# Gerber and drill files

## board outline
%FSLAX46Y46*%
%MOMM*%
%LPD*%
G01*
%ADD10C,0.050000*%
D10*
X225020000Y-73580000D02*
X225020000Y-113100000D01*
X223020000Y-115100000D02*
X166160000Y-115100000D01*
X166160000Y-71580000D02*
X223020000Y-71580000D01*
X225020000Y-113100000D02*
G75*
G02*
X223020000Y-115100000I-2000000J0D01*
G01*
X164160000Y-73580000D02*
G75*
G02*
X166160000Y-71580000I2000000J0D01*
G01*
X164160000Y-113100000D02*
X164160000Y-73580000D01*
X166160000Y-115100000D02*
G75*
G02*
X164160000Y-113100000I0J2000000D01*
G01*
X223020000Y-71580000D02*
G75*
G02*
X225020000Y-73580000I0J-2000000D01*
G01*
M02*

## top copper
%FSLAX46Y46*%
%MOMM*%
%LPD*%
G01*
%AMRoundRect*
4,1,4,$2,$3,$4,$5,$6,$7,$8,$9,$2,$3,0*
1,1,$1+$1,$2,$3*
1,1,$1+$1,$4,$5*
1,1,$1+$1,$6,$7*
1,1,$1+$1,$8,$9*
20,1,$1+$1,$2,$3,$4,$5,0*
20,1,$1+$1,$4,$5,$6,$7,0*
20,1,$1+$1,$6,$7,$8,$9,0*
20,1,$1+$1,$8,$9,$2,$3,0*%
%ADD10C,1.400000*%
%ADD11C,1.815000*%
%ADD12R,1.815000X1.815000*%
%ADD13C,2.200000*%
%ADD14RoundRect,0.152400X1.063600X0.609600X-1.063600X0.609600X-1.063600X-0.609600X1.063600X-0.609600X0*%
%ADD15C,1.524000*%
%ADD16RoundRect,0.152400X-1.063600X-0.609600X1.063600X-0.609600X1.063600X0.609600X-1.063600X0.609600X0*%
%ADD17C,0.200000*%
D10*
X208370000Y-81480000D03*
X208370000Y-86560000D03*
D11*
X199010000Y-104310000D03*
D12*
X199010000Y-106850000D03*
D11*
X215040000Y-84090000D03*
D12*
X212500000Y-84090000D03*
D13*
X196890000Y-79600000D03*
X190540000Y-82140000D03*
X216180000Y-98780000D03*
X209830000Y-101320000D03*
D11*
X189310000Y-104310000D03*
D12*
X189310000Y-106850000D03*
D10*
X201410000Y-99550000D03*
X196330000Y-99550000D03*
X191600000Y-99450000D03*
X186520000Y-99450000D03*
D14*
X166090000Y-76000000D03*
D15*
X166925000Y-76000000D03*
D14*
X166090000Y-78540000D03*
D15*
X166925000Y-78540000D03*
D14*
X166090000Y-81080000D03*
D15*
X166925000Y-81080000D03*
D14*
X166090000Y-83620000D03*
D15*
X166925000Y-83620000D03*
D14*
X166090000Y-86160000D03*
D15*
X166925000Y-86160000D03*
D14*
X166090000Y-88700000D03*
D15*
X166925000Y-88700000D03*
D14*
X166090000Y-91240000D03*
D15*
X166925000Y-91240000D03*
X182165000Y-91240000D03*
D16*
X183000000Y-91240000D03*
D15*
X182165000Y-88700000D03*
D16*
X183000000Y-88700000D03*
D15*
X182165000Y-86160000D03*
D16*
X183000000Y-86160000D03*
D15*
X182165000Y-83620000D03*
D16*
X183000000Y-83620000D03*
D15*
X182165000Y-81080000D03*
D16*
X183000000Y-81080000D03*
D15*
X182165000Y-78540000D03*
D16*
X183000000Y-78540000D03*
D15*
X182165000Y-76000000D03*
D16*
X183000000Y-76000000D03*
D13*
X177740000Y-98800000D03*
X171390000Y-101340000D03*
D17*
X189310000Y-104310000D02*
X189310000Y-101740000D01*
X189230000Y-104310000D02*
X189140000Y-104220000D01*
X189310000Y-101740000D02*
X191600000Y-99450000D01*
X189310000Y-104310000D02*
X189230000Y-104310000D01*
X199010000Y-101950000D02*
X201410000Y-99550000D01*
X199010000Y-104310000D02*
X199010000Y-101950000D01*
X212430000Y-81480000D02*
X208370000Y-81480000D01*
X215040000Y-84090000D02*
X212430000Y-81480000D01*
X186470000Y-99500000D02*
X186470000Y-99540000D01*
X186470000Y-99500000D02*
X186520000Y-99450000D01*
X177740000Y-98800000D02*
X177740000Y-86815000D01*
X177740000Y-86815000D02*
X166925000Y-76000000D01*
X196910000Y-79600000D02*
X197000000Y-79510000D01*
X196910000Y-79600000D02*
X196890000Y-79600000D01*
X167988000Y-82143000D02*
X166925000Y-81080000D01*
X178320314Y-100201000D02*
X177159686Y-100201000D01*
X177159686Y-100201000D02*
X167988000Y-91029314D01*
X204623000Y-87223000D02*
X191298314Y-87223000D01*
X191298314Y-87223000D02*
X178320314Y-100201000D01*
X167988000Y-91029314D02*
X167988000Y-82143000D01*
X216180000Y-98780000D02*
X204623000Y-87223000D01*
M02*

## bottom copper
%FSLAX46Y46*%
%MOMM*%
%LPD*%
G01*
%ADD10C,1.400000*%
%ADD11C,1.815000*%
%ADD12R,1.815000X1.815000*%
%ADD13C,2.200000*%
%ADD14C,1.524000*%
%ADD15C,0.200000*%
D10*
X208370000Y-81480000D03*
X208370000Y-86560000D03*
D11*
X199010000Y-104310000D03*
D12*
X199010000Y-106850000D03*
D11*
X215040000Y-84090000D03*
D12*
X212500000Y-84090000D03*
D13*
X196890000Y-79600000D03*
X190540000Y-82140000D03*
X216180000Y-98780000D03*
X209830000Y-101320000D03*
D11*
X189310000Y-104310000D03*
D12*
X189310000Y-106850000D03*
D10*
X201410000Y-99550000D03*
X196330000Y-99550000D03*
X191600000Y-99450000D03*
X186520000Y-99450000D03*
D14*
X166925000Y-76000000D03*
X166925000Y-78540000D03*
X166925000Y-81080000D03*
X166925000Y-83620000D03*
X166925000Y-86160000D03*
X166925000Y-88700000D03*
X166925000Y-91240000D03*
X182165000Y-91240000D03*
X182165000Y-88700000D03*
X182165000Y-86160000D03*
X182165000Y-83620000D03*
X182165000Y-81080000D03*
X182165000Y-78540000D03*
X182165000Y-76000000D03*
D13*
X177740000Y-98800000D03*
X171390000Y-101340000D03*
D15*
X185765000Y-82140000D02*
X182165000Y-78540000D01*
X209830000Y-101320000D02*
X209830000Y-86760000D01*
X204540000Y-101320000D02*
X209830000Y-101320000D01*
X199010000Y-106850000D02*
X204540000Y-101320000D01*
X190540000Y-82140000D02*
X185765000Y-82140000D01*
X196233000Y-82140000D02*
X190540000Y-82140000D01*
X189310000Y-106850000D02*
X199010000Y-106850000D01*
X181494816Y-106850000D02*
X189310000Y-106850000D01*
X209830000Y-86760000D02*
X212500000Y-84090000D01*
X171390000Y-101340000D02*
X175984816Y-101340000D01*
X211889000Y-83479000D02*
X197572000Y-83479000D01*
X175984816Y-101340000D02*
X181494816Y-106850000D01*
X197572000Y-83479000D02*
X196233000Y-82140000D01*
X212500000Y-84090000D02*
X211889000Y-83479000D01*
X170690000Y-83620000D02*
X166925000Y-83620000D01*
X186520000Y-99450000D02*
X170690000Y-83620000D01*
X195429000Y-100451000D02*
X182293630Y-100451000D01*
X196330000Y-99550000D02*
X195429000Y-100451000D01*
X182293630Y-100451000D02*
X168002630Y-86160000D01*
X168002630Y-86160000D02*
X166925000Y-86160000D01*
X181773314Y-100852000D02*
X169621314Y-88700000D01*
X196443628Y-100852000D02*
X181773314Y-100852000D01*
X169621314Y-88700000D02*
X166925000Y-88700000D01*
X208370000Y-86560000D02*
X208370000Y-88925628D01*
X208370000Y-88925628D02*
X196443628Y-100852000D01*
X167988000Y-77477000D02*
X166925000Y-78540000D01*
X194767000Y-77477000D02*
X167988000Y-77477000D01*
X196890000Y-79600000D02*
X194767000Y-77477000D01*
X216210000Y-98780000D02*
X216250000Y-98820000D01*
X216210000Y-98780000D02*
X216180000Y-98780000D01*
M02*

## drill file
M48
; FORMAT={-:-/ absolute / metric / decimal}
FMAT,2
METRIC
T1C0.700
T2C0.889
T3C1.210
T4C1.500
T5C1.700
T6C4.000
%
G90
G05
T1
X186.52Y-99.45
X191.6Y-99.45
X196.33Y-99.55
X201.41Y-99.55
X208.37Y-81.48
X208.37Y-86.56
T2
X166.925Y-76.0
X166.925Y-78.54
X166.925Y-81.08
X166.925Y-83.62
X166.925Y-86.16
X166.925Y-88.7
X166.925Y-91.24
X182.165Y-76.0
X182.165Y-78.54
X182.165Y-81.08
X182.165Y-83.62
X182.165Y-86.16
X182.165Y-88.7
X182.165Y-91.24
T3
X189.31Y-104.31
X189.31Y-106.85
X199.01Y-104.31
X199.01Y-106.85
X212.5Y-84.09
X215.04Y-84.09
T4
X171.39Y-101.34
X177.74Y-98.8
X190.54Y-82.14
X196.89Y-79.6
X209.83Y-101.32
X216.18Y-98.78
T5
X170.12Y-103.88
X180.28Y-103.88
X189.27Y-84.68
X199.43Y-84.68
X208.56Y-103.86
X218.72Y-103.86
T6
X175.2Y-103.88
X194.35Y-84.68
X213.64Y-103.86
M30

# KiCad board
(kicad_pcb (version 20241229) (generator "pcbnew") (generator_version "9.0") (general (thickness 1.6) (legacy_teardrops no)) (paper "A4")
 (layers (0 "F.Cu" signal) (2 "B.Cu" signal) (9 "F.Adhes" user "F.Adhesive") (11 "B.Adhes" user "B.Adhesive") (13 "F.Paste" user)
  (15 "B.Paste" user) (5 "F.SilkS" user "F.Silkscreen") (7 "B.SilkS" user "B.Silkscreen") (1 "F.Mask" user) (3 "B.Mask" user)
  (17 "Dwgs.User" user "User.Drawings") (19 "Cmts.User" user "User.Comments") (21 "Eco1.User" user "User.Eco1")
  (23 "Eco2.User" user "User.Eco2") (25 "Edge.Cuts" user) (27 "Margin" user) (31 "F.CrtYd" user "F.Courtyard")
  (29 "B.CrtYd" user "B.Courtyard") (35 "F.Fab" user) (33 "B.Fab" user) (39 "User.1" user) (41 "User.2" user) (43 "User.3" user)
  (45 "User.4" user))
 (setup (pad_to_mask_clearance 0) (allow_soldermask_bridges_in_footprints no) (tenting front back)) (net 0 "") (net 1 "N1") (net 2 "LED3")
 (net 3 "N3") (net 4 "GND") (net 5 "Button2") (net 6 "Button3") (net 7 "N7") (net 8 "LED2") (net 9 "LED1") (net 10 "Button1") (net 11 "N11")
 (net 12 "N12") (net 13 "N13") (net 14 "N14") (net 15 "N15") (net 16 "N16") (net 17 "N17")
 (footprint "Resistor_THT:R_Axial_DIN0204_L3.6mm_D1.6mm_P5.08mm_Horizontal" (layer "F.Cu") (at 208.37 81.48 -90)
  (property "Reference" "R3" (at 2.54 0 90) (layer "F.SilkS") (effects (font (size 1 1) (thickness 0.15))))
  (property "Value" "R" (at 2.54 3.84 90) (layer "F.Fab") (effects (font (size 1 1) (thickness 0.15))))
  (pad "1" thru_hole circle (at 0 0 270) (size 1.4 1.4) (drill 0.7) (layers "*.Cu" "*.Mask") (remove_unused_layers no) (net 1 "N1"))
  (pad "2" thru_hole circle (at 5.08 0 270) (size 1.4 1.4) (drill 0.7) (layers "*.Cu" "*.Mask") (remove_unused_layers no) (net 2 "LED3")))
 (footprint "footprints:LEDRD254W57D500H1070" (layer "F.Cu") (at 199.01 105.58 90)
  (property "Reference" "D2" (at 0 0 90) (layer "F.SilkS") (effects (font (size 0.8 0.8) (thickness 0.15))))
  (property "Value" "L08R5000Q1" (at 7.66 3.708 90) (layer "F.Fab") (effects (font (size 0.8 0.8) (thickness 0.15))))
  (pad "A" thru_hole circle (at 1.27 0 90) (size 1.815 1.815) (drill 1.21) (layers "*.Cu" "*.Mask") (remove_unused_layers no) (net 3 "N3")
   (solder_mask_margin 0.102))
  (pad "C" thru_hole rect (at -1.27 0 90) (size 1.815 1.815) (drill 1.21) (layers "*.Cu" "*.Mask") (remove_unused_layers no) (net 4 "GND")
   (solder_mask_margin 0.102)))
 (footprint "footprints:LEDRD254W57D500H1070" (layer "F.Cu") (at 213.77 84.09)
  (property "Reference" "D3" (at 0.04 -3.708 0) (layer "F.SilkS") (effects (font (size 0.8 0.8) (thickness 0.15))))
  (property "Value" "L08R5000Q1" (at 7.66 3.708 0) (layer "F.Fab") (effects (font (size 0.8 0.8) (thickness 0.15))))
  (pad "A" thru_hole circle (at 1.27 0) (size 1.815 1.815) (drill 1.21) (layers "*.Cu" "*.Mask") (remove_unused_layers no) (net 1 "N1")
   (solder_mask_margin 0.102))
  (pad "C" thru_hole rect (at -1.27 0) (size 1.815 1.815) (drill 1.21) (layers "*.Cu" "*.Mask") (remove_unused_layers no) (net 4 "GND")
   (solder_mask_margin 0.102)))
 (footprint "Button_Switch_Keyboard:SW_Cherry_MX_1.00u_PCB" (layer "F.Cu") (at 196.89 79.6)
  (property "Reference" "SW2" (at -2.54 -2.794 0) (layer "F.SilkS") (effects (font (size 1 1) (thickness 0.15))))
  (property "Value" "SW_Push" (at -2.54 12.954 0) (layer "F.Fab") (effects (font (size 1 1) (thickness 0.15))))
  (pad "" np_thru_hole circle (at -7.62 5.08) (size 1.7 1.7) (drill 1.7) (layers "*.Cu" "*.Mask"))
  (pad "" np_thru_hole circle (at -2.54 5.08) (size 4 4) (drill 4) (layers "*.Cu" "*.Mask"))
  (pad "" np_thru_hole circle (at 2.54 5.08) (size 1.7 1.7) (drill 1.7) (layers "*.Cu" "*.Mask"))
  (pad "1" thru_hole circle (at 0 0) (size 2.2 2.2) (drill 1.5) (layers "*.Cu" "*.Mask") (remove_unused_layers no) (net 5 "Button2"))
  (pad "2" thru_hole circle (at -6.35 2.54) (size 2.2 2.2) (drill 1.5) (layers "*.Cu" "*.Mask") (remove_unused_layers no) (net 4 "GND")))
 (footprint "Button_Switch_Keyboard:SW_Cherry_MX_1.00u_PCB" (layer "F.Cu") (at 216.18 98.78)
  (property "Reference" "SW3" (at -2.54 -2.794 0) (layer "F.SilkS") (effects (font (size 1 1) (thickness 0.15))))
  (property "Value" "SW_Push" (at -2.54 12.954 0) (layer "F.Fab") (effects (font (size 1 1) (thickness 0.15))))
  (pad "" np_thru_hole circle (at -7.62 5.08) (size 1.7 1.7) (drill 1.7) (layers "*.Cu" "*.Mask"))
  (pad "" np_thru_hole circle (at -2.54 5.08) (size 4 4) (drill 4) (layers "*.Cu" "*.Mask"))
  (pad "" np_thru_hole circle (at 2.54 5.08) (size 1.7 1.7) (drill 1.7) (layers "*.Cu" "*.Mask"))
  (pad "1" thru_hole circle (at 0 0) (size 2.2 2.2) (drill 1.5) (layers "*.Cu" "*.Mask") (remove_unused_layers no) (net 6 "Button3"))
  (pad "2" thru_hole circle (at -6.35 2.54) (size 2.2 2.2) (drill 1.5) (layers "*.Cu" "*.Mask") (remove_unused_layers no) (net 4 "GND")))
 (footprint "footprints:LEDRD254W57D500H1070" (layer "F.Cu") (at 189.31 105.58 90)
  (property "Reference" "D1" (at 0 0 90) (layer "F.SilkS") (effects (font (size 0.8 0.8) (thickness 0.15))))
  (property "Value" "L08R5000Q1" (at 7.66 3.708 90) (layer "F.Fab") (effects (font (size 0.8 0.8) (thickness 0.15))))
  (pad "A" thru_hole circle (at 1.27 0 90) (size 1.815 1.815) (drill 1.21) (layers "*.Cu" "*.Mask") (remove_unused_layers no) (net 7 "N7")
   (solder_mask_margin 0.102))
  (pad "C" thru_hole rect (at -1.27 0 90) (size 1.815 1.815) (drill 1.21) (layers "*.Cu" "*.Mask") (remove_unused_layers no) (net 4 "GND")
   (solder_mask_margin 0.102)))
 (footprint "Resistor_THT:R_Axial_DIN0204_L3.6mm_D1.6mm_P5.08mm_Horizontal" (layer "F.Cu") (at 201.41 99.55 180)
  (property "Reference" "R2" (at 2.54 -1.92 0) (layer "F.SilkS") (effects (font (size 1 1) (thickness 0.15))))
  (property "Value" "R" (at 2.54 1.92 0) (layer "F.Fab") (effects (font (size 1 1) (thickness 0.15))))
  (pad "1" thru_hole circle (at 0 0 180) (size 1.4 1.4) (drill 0.7) (layers "*.Cu" "*.Mask") (remove_unused_layers no) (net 3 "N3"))
  (pad "2" thru_hole circle (at 5.08 0 180) (size 1.4 1.4) (drill 0.7) (layers "*.Cu" "*.Mask") (remove_unused_layers no) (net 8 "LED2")))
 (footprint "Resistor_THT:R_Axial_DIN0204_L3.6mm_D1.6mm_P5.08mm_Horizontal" (layer "F.Cu") (at 191.6 99.45 180)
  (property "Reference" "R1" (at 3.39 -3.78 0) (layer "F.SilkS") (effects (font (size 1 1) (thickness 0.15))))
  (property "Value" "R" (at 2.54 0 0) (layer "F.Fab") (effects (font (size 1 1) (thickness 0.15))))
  (pad "1" thru_hole circle (at 0 0 180) (size 1.4 1.4) (drill 0.7) (layers "*.Cu" "*.Mask") (remove_unused_layers no) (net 7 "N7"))
  (pad "2" thru_hole circle (at 5.08 0 180) (size 1.4 1.4) (drill 0.7) (layers "*.Cu" "*.Mask") (remove_unused_layers no) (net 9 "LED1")))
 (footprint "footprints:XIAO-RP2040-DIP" (layer "F.Cu") (at 174.545 83.62)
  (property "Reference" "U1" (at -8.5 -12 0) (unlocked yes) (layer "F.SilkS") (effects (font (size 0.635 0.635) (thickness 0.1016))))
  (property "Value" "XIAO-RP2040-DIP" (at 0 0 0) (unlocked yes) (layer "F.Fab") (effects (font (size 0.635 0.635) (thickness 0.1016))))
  (pad "1" smd roundrect (at -8.455 -7.62 180) (size 2.432 1.524) (layers "F.Cu" "F.Mask") (roundrect_rratio 0.1) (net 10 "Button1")
   (thermal_bridge_angle 45))
  (pad "1" thru_hole circle (at -7.62 -7.62 180) (size 1.524 1.524) (drill 0.889) (layers "*.Cu" "*.Mask") (remove_unused_layers no)
   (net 10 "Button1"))
  (pad "2" smd roundrect (at -8.455 -5.08 180) (size 2.432 1.524) (layers "F.Cu" "F.Mask") (roundrect_rratio 0.1) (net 5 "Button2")
   (thermal_bridge_angle 45))
  (pad "2" thru_hole circle (at -7.62 -5.08 180) (size 1.524 1.524) (drill 0.889) (layers "*.Cu" "*.Mask") (remove_unused_layers no)
   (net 5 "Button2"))
  (pad "3" smd roundrect (at -8.455 -2.54 180) (size 2.432 1.524) (layers "F.Cu" "F.Mask") (roundrect_rratio 0.1) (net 6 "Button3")
   (thermal_bridge_angle 45))
  (pad "3" thru_hole circle (at -7.62 -2.54 180) (size 1.524 1.524) (drill 0.889) (layers "*.Cu" "*.Mask") (remove_unused_layers no)
   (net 6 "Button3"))
  (pad "4" smd roundrect (at -8.455 0 180) (size 2.432 1.524) (layers "F.Cu" "F.Mask") (roundrect_rratio 0.1) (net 9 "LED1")
   (thermal_bridge_angle 45))
  (pad "4" thru_hole circle (at -7.62 0 180) (size 1.524 1.524) (drill 0.889) (layers "*.Cu" "*.Mask") (remove_unused_layers no)
   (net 9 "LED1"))
  (pad "5" smd roundrect (at -8.455 2.54 180) (size 2.432 1.524) (layers "F.Cu" "F.Mask") (roundrect_rratio 0.1) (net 8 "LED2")
   (thermal_bridge_angle 45))
  (pad "5" thru_hole circle (at -7.62 2.54 180) (size 1.524 1.524) (drill 0.889) (layers "*.Cu" "*.Mask") (remove_unused_layers no)
   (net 8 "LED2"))
  (pad "6" smd roundrect (at -8.455 5.08 180) (size 2.432 1.524) (layers "F.Cu" "F.Mask") (roundrect_rratio 0.1) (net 2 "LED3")
   (thermal_bridge_angle 45))
  (pad "6" thru_hole circle (at -7.62 5.08 180) (size 1.524 1.524) (drill 0.889) (layers "*.Cu" "*.Mask") (remove_unused_layers no)
   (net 2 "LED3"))
  (pad "7" smd roundrect (at -8.455 7.62 180) (size 2.432 1.524) (layers "F.Cu" "F.Mask") (roundrect_rratio 0.1) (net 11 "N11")
   (thermal_bridge_angle 45))
  (pad "7" thru_hole circle (at -7.62 7.62 180) (size 1.524 1.524) (drill 0.889) (layers "*.Cu" "*.Mask") (remove_unused_layers no)
   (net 11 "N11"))
  (pad "8" thru_hole circle (at 7.62 7.62) (size 1.524 1.524) (drill 0.889) (layers "*.Cu" "*.Mask") (remove_unused_layers no)
   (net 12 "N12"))
  (pad "8" smd roundrect (at 8.455 7.62) (size 2.432 1.524) (layers "F.Cu" "F.Mask") (roundrect_rratio 0.1) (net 12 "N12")
   (thermal_bridge_angle 45))
  (pad "9" thru_hole circle (at 7.62 5.08) (size 1.524 1.524) (drill 0.889) (layers "*.Cu" "*.Mask") (remove_unused_layers no)
   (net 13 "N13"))
  (pad "9" smd roundrect (at 8.455 5.08) (size 2.432 1.524) (layers "F.Cu" "F.Mask") (roundrect_rratio 0.1) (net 13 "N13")
   (thermal_bridge_angle 45))
  (pad "10" thru_hole circle (at 7.62 2.54) (size 1.524 1.524) (drill 0.889) (layers "*.Cu" "*.Mask") (remove_unused_layers no)
   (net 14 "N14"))
  (pad "10" smd roundrect (at 8.455 2.54) (size 2.432 1.524) (layers "F.Cu" "F.Mask") (roundrect_rratio 0.1) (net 14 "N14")
   (thermal_bridge_angle 45))
  (pad "11" thru_hole circle (at 7.62 0) (size 1.524 1.524) (drill 0.889) (layers "*.Cu" "*.Mask") (remove_unused_layers no) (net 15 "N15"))
  (pad "11" smd roundrect (at 8.455 0) (size 2.432 1.524) (layers "F.Cu" "F.Mask") (roundrect_rratio 0.1) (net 15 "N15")
   (thermal_bridge_angle 45))
  (pad "12" thru_hole circle (at 7.62 -2.54) (size 1.524 1.524) (drill 0.889) (layers "*.Cu" "*.Mask") (remove_unused_layers no)
   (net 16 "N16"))
  (pad "12" smd roundrect (at 8.455 -2.54) (size 2.432 1.524) (layers "F.Cu" "F.Mask") (roundrect_rratio 0.1) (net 16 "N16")
   (thermal_bridge_angle 45))
  (pad "13" thru_hole circle (at 7.62 -5.08) (size 1.524 1.524) (drill 0.889) (layers "*.Cu" "*.Mask") (remove_unused_layers no)
   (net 4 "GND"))
  (pad "13" smd roundrect (at 8.455 -5.08) (size 2.432 1.524) (layers "F.Cu" "F.Mask") (roundrect_rratio 0.1) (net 4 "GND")
   (thermal_bridge_angle 45))
  (pad "14" thru_hole circle (at 7.62 -7.62) (size 1.524 1.524) (drill 0.889) (layers "*.Cu" "*.Mask") (remove_unused_layers no)
   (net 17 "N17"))
  (pad "14" smd roundrect (at 8.455 -7.62) (size 2.432 1.524) (layers "F.Cu" "F.Mask") (roundrect_rratio 0.1) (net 17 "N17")
   (thermal_bridge_angle 45)))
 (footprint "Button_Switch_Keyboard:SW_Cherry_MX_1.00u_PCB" (layer "F.Cu") (at 177.74 98.8)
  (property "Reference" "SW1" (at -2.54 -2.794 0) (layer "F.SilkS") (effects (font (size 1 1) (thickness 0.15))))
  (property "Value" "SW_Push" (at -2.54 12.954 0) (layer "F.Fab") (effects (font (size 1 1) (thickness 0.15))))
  (pad "" np_thru_hole circle (at -7.62 5.08) (size 1.7 1.7) (drill 1.7) (layers "*.Cu" "*.Mask"))
  (pad "" np_thru_hole circle (at -2.54 5.08) (size 4 4) (drill 4) (layers "*.Cu" "*.Mask"))
  (pad "" np_thru_hole circle (at 2.54 5.08) (size 1.7 1.7) (drill 1.7) (layers "*.Cu" "*.Mask"))
  (pad "1" thru_hole circle (at 0 0) (size 2.2 2.2) (drill 1.5) (layers "*.Cu" "*.Mask") (remove_unused_layers no) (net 10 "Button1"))
  (pad "2" thru_hole circle (at -6.35 2.54) (size 2.2 2.2) (drill 1.5) (layers "*.Cu" "*.Mask") (remove_unused_layers no) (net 4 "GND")))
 (gr_line (start 225.02 73.58) (end 225.02 113.1) (stroke (width 0.05) (type default)) (layer "Edge.Cuts"))
 (gr_line (start 223.02 115.1) (end 166.16 115.1) (stroke (width 0.05) (type default)) (layer "Edge.Cuts"))
 (gr_line (start 166.16 71.58) (end 223.02 71.58) (stroke (width 0.05) (type default)) (layer "Edge.Cuts"))
 (gr_arc (start 225.02 113.1) (mid 224.434214 114.514214) (end 223.02 115.1) (stroke (width 0.05) (type default)) (layer "Edge.Cuts"))
 (gr_arc (start 164.16 73.58) (mid 164.745786 72.165786) (end 166.16 71.58) (stroke (width 0.05) (type default)) (layer "Edge.Cuts"))
 (gr_line (start 164.16 113.1) (end 164.16 73.58) (stroke (width 0.05) (type default)) (layer "Edge.Cuts"))
 (gr_arc (start 166.16 115.1) (mid 164.745786 114.514214) (end 164.16 113.1) (stroke (width 0.05) (type default)) (layer "Edge.Cuts"))
 (gr_arc (start 223.02 71.58) (mid 224.434214 72.165786) (end 225.02 73.58) (stroke (width 0.05) (type default)) (layer "Edge.Cuts"))
 (segment (start 185.765 82.14) (end 182.165 78.54) (width 0.2) (layer "B.Cu") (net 4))
 (segment (start 209.83 101.32) (end 209.83 86.76) (width 0.2) (layer "B.Cu") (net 4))
 (segment (start 204.54 101.32) (end 209.83 101.32) (width 0.2) (layer "B.Cu") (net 4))
 (segment (start 199.01 106.85) (end 204.54 101.32) (width 0.2) (layer "B.Cu") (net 4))
 (segment (start 190.54 82.14) (end 185.765 82.14) (width 0.2) (layer "B.Cu") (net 4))
 (segment (start 196.233 82.14) (end 190.54 82.14) (width 0.2) (layer "B.Cu") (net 4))
 (segment (start 189.31 106.85) (end 199.01 106.85) (width 0.2) (layer "B.Cu") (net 4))
 (segment (start 181.494816 106.85) (end 189.31 106.85) (width 0.2) (layer "B.Cu") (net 4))
 (segment (start 209.83 86.76) (end 212.5 84.09) (width 0.2) (layer "B.Cu") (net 4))
 (segment (start 171.39 101.34) (end 175.984816 101.34) (width 0.2) (layer "B.Cu") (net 4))
 (segment (start 211.889 83.479) (end 197.572 83.479) (width 0.2) (layer "B.Cu") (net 4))
 (segment (start 175.984816 101.34) (end 181.494816 106.85) (width 0.2) (layer "B.Cu") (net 4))
 (segment (start 197.572 83.479) (end 196.233 82.14) (width 0.2) (layer "B.Cu") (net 4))
 (segment (start 212.5 84.09) (end 211.889 83.479) (width 0.2) (layer "B.Cu") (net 4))
 (segment (start 189.31 104.31) (end 189.31 101.74) (width 0.2) (layer "F.Cu") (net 7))
 (segment (start 189.23 104.31) (end 189.14 104.22) (width 0.2) (layer "F.Cu") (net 7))
 (segment (start 189.31 101.74) (end 191.6 99.45) (width 0.2) (layer "F.Cu") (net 7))
 (segment (start 189.31 104.31) (end 189.23 104.31) (width 0.2) (layer "F.Cu") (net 7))
 (segment (start 199.01 101.95) (end 201.41 99.55) (width 0.2) (layer "F.Cu") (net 3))
 (segment (start 199.01 104.31) (end 199.01 101.95) (width 0.2) (layer "F.Cu") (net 3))
 (segment (start 212.43 81.48) (end 208.37 81.48) (width 0.2) (layer "F.Cu") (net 1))
 (segment (start 215.04 84.09) (end 212.43 81.48) (width 0.2) (layer "F.Cu") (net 1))
 (segment (start 186.47 99.5) (end 186.47 99.54) (width 0.2) (layer "F.Cu") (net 9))
 (segment (start 186.47 99.5) (end 186.52 99.45) (width 0.2) (layer "F.Cu") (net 9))
 (segment (start 170.69 83.62) (end 166.925 83.62) (width 0.2) (layer "B.Cu") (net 9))
 (segment (start 186.52 99.45) (end 170.69 83.62) (width 0.2) (layer "B.Cu") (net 9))
 (segment (start 195.429 100.451) (end 182.29363 100.451) (width 0.2) (layer "B.Cu") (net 8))
 (segment (start 196.33 99.55) (end 195.429 100.451) (width 0.2) (layer "B.Cu") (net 8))
 (segment (start 182.29363 100.451) (end 168.00263 86.16) (width 0.2) (layer "B.Cu") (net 8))
 (segment (start 168.00263 86.16) (end 166.925 86.16) (width 0.2) (layer "B.Cu") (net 8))
 (segment (start 181.773314 100.852) (end 169.621314 88.7) (width 0.2) (layer "B.Cu") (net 2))
 (segment (start 196.443628 100.852) (end 181.773314 100.852) (width 0.2) (layer "B.Cu") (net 2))
 (segment (start 169.621314 88.7) (end 166.925 88.7) (width 0.2) (layer "B.Cu") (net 2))
 (segment (start 208.37 86.56) (end 208.37 88.925628) (width 0.2) (layer "B.Cu") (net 2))
 (segment (start 208.37 88.925628) (end 196.443628 100.852) (width 0.2) (layer "B.Cu") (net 2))
 (segment (start 177.74 98.8) (end 177.74 86.815) (width 0.2) (layer "F.Cu") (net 10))
 (segment (start 177.74 86.815) (end 166.925 76) (width 0.2) (layer "F.Cu") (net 10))
 (segment (start 196.91 79.6) (end 197 79.51) (width 0.2) (layer "F.Cu") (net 5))
 (segment (start 196.91 79.6) (end 196.89 79.6) (width 0.2) (layer "F.Cu") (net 5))
 (segment (start 167.988 77.477) (end 166.925 78.54) (width 0.2) (layer "B.Cu") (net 5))
 (segment (start 194.767 77.477) (end 167.988 77.477) (width 0.2) (layer "B.Cu") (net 5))
 (segment (start 196.89 79.6) (end 194.767 77.477) (width 0.2) (layer "B.Cu") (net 5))
 (segment (start 167.988 82.143) (end 166.925 81.08) (width 0.2) (layer "F.Cu") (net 6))
 (segment (start 178.320314 100.201) (end 177.159686 100.201) (width 0.2) (layer "F.Cu") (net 6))
 (segment (start 177.159686 100.201) (end 167.988 91.029314) (width 0.2) (layer "F.Cu") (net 6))
 (segment (start 204.623 87.223) (end 191.298314 87.223) (width 0.2) (layer "F.Cu") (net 6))
 (segment (start 191.298314 87.223) (end 178.320314 100.201) (width 0.2) (layer "F.Cu") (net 6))
 (segment (start 167.988 91.029314) (end 167.988 82.143) (width 0.2) (layer "F.Cu") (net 6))
 (segment (start 216.18 98.78) (end 204.623 87.223) (width 0.2) (layer "F.Cu") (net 6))
 (segment (start 216.21 98.78) (end 216.25 98.82) (width 0.2) (layer "B.Cu") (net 6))
 (segment (start 216.21 98.78) (end 216.18 98.78) (width 0.2) (layer "B.Cu") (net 6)))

